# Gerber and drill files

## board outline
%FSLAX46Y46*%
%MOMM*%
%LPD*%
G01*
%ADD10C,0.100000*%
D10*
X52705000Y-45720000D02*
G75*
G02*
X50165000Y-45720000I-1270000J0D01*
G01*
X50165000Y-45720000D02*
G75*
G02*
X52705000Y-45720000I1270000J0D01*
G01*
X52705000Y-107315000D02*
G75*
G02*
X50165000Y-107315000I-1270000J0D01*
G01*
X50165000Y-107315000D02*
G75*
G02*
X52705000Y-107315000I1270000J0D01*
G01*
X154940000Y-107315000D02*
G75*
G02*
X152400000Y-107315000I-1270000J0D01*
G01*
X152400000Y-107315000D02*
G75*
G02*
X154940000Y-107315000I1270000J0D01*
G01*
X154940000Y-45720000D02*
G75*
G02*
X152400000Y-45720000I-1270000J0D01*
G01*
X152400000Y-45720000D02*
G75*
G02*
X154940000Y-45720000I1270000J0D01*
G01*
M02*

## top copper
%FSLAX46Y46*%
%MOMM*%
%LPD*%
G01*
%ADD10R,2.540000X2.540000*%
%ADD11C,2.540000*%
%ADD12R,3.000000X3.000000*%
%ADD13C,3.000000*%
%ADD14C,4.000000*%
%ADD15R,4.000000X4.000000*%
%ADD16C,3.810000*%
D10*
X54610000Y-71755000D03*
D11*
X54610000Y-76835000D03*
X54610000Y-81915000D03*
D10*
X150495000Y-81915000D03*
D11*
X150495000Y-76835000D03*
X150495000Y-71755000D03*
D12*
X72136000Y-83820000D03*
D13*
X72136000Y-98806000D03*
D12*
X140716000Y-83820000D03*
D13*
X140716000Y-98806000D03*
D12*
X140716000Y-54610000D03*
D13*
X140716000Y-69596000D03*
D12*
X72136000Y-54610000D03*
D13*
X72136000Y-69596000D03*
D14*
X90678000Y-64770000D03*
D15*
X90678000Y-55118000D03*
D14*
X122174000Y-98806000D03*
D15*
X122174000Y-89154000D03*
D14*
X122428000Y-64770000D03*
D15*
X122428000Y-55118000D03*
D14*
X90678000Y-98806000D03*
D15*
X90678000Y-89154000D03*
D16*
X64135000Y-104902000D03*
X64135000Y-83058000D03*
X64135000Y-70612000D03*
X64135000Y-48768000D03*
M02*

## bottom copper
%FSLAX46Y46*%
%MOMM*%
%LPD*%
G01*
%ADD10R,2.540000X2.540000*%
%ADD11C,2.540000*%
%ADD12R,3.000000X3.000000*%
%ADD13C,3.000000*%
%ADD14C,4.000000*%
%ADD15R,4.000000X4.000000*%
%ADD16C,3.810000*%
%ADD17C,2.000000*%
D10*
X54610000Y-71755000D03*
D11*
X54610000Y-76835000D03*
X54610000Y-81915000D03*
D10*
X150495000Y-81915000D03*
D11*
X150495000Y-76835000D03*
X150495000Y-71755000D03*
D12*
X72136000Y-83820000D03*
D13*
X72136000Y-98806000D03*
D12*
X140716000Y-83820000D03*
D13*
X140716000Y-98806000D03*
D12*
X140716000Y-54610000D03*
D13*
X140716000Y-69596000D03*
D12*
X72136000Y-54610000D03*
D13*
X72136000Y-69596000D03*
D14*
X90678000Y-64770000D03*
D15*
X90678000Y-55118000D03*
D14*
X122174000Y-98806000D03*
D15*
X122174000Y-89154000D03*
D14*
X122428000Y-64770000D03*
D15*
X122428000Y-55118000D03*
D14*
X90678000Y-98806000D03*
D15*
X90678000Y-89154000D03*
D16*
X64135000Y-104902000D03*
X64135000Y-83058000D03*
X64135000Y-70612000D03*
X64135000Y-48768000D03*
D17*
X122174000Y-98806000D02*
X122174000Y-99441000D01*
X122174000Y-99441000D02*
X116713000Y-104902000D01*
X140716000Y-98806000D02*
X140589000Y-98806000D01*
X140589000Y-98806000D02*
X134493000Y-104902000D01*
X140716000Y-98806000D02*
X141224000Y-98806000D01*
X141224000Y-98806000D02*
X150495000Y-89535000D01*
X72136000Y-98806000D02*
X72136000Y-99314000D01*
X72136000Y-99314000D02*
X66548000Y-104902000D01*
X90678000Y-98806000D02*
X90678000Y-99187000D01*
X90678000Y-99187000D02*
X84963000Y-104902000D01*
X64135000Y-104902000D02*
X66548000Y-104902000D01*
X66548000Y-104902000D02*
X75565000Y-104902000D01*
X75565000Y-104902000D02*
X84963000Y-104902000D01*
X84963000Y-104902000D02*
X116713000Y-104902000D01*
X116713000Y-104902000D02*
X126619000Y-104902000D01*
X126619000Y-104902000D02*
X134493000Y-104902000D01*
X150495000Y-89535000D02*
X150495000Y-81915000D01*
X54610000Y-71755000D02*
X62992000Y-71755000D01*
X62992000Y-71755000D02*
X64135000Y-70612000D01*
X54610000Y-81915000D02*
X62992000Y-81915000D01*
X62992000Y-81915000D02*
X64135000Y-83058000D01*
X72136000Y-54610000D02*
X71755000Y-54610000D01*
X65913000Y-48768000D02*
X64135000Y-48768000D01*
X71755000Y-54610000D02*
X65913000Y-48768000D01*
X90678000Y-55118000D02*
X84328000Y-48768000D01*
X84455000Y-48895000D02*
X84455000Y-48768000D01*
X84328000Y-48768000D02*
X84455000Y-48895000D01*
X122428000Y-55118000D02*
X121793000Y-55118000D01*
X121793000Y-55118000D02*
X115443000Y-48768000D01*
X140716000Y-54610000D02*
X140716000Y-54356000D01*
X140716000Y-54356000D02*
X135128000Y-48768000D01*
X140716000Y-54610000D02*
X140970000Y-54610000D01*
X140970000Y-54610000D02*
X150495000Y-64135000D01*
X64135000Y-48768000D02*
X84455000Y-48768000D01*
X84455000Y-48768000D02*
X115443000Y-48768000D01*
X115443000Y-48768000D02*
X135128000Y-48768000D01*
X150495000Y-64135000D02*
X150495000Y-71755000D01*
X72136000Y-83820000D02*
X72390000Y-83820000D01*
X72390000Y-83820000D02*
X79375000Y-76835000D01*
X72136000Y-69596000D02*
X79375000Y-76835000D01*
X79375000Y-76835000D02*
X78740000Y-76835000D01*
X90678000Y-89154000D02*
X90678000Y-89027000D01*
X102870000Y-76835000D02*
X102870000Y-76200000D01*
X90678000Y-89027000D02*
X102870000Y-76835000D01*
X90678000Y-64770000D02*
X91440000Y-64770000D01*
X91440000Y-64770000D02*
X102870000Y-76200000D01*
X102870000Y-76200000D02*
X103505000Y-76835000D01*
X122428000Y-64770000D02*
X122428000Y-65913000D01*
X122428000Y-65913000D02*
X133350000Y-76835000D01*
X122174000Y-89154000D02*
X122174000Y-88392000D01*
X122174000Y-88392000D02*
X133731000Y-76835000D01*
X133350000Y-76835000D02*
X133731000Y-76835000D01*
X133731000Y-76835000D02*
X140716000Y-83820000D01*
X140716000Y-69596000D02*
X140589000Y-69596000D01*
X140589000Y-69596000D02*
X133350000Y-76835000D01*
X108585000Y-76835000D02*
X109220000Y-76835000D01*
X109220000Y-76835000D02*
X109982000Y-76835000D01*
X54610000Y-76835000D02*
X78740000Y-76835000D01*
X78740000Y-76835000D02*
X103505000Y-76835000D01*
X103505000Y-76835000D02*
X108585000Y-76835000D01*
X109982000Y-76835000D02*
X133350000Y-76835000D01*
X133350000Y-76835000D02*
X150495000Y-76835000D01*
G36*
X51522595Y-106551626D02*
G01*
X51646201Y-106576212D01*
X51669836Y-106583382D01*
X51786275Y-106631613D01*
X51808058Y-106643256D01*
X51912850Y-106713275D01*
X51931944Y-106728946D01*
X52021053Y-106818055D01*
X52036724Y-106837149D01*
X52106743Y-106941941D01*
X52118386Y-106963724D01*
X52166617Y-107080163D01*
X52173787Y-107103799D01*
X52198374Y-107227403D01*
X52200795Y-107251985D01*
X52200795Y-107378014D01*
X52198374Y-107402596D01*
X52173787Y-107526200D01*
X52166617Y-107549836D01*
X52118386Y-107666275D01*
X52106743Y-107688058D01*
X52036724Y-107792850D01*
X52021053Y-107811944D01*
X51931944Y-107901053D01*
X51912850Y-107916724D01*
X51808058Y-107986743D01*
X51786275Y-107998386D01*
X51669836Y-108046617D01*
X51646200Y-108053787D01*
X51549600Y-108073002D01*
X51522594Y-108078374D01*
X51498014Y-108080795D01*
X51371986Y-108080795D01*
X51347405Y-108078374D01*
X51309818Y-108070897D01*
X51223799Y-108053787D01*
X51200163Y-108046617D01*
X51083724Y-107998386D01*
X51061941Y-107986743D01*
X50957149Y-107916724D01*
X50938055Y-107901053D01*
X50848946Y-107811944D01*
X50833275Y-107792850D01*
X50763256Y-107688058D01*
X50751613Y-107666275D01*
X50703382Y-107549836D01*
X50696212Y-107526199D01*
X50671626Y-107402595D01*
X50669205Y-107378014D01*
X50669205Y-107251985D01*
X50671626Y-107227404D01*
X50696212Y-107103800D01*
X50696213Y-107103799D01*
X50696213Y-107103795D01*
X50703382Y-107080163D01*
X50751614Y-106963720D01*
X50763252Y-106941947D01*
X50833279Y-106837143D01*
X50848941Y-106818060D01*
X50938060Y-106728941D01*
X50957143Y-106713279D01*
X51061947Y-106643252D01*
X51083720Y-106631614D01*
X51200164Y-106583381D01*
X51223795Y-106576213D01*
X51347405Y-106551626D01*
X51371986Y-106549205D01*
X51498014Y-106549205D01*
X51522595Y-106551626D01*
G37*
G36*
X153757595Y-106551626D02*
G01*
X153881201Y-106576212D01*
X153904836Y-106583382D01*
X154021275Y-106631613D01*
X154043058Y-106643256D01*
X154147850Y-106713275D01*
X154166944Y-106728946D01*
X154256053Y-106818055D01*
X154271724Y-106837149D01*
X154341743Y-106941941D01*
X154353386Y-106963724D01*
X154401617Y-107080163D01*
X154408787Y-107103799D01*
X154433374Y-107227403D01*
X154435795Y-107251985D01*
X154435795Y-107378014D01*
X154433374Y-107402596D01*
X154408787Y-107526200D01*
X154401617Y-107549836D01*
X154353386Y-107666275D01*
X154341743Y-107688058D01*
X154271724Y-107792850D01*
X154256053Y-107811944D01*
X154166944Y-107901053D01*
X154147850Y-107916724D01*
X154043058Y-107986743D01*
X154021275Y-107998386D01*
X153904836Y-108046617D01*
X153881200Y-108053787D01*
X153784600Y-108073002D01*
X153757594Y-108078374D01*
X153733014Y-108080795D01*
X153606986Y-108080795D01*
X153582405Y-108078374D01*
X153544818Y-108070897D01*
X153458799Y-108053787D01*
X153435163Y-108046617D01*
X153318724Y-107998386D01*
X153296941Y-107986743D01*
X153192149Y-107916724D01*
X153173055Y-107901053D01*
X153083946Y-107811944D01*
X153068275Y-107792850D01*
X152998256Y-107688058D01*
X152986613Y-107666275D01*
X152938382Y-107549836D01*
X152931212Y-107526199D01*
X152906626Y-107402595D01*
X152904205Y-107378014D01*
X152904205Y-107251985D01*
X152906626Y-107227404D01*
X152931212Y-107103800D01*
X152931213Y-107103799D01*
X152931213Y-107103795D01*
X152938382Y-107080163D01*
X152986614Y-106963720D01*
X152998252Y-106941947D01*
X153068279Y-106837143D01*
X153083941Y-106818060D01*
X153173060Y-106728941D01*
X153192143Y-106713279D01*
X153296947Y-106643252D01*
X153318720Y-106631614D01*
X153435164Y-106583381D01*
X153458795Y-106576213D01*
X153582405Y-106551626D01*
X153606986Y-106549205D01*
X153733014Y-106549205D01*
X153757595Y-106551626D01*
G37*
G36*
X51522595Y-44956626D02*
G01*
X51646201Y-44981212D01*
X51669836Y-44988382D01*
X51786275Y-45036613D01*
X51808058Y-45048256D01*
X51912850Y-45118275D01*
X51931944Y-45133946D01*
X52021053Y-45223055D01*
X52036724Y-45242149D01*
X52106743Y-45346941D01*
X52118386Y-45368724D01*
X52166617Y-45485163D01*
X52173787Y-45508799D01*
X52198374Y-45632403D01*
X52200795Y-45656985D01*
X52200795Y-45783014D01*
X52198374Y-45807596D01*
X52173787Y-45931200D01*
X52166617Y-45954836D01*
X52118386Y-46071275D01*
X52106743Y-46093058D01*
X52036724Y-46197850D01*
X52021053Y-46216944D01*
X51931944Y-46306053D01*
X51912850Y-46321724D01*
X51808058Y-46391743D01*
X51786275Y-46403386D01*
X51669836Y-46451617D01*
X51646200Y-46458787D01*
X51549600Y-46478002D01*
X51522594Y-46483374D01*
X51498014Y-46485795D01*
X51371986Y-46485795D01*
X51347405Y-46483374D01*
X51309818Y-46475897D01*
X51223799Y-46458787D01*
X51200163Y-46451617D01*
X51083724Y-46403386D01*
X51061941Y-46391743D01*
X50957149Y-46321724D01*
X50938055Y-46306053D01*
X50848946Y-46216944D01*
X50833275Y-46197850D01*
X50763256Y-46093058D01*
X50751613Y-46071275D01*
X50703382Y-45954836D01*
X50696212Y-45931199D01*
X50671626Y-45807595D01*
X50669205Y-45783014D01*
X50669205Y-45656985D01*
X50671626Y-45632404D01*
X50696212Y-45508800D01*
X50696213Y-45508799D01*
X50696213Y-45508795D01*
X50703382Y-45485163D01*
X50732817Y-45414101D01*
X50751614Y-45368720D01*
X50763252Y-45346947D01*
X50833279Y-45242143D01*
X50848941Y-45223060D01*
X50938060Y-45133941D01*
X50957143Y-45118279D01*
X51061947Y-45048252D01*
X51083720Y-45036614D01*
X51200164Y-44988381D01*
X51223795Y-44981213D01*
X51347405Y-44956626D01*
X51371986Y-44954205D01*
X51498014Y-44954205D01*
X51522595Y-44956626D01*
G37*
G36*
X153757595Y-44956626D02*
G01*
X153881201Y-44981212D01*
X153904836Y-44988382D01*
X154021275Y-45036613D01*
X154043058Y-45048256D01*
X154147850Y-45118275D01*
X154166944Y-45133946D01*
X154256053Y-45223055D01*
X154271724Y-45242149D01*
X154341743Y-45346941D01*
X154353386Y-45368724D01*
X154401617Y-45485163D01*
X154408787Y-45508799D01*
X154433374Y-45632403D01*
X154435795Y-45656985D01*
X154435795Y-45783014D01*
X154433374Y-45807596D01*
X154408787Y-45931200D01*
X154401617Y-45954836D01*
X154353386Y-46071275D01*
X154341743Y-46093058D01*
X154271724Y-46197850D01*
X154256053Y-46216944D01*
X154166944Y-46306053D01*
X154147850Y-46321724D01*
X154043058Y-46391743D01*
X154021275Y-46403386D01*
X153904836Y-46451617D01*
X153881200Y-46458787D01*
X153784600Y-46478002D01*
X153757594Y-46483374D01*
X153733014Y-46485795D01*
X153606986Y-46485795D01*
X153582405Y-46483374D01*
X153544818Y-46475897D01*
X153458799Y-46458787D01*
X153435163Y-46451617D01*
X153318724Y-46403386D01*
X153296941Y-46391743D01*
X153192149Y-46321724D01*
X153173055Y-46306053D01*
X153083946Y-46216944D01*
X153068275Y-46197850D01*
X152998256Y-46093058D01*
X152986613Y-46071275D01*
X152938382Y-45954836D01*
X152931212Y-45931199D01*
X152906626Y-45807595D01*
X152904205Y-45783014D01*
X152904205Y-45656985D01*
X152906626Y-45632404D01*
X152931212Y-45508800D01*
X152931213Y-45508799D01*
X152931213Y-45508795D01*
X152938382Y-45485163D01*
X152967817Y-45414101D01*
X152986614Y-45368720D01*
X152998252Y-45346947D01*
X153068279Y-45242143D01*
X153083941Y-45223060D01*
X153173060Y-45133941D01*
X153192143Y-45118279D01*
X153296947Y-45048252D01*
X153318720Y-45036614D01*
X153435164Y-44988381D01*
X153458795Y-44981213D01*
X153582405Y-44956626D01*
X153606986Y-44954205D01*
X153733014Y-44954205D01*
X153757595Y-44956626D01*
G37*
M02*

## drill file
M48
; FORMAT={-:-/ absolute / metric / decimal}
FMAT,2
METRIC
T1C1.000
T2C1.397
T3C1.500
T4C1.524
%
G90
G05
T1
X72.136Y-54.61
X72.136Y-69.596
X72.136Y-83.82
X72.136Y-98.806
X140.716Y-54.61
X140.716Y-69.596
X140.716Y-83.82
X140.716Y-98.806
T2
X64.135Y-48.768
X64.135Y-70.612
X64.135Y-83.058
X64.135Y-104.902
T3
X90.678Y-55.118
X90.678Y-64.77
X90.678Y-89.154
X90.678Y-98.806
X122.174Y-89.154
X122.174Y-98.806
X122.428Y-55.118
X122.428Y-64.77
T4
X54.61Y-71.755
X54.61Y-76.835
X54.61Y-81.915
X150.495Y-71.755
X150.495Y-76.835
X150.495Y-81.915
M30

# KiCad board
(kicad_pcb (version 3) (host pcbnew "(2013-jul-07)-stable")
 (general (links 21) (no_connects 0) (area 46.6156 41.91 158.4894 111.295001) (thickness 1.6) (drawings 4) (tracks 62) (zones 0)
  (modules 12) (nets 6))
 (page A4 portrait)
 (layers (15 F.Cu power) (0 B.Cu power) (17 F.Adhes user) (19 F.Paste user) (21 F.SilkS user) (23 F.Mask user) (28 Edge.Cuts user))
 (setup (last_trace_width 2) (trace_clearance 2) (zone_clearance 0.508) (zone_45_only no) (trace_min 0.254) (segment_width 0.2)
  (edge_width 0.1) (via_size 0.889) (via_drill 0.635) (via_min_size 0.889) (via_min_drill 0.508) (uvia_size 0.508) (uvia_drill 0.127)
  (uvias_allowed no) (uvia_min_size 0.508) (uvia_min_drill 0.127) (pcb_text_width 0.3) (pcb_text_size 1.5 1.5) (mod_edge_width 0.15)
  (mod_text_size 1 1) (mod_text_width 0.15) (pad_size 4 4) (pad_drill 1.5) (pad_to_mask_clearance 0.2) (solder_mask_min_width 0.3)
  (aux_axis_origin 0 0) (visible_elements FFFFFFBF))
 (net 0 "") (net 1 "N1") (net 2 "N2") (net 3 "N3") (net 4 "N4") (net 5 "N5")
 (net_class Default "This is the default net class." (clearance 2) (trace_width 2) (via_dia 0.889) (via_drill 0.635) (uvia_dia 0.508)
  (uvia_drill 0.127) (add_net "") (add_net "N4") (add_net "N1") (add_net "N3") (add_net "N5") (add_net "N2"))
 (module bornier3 (layer F.Cu) (at 54.61 76.835 270)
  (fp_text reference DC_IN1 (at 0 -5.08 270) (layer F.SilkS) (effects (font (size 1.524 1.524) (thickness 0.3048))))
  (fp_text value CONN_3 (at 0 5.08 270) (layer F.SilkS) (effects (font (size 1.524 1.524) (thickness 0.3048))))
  (pad 1 thru_hole rect (at -5.08 0 270) (size 2.54 2.54) (drill 1.524) (layers *.Cu *.Mask F.SilkS) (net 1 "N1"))
  (pad 2 thru_hole circle (at 0 0 270) (size 2.54 2.54) (drill 1.524) (layers *.Cu *.Mask F.SilkS) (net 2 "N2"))
  (pad 3 thru_hole circle (at 5.08 0 270) (size 2.54 2.54) (drill 1.524) (layers *.Cu *.Mask F.SilkS) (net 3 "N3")))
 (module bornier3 (layer F.Cu) (at 150.495 76.835 90)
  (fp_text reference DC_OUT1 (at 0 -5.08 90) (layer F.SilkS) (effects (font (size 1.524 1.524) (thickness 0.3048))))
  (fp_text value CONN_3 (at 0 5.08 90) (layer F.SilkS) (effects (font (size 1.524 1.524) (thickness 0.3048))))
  (pad 1 thru_hole rect (at -5.08 0 90) (size 2.54 2.54) (drill 1.524) (layers *.Cu *.Mask F.SilkS) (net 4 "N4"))
  (pad 2 thru_hole circle (at 0 0 90) (size 2.54 2.54) (drill 1.524) (layers *.Cu *.Mask F.SilkS) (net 2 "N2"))
  (pad 3 thru_hole circle (at 5.08 0 90) (size 2.54 2.54) (drill 1.524) (layers *.Cu *.Mask F.SilkS) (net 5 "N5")))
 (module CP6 (layer F.Cu) (at 72.136 91.44 270)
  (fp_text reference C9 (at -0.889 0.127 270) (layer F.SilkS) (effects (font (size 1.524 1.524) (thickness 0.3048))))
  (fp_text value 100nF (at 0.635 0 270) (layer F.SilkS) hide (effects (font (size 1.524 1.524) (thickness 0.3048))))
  (pad 1 thru_hole rect (at -7.62 0 270) (size 3 3) (drill 1) (layers *.Cu *.Mask F.SilkS) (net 2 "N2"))
  (pad 2 thru_hole circle (at 7.366 0 270) (size 3 3) (drill 1) (layers *.Cu *.Mask F.SilkS) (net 4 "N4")))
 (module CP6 (layer F.Cu) (at 140.716 91.44 270)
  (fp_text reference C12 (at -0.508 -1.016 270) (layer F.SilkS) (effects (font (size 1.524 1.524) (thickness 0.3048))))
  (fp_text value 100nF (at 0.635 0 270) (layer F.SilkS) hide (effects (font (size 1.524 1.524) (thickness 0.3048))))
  (pad 1 thru_hole rect (at -7.62 0 270) (size 3 3) (drill 1) (layers *.Cu *.Mask F.SilkS) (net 2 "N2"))
  (pad 2 thru_hole circle (at 7.366 0 270) (size 3 3) (drill 1) (layers *.Cu *.Mask F.SilkS) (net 4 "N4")))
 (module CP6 (layer F.Cu) (at 140.716 62.23 270)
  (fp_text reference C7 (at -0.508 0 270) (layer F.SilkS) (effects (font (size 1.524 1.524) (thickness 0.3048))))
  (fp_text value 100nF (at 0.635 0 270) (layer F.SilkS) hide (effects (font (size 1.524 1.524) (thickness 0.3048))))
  (pad 1 thru_hole rect (at -7.62 0 270) (size 3 3) (drill 1) (layers *.Cu *.Mask F.SilkS) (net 5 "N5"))
  (pad 2 thru_hole circle (at 7.366 0 270) (size 3 3) (drill 1) (layers *.Cu *.Mask F.SilkS) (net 2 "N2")))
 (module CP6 (layer F.Cu) (at 72.136 62.23 270)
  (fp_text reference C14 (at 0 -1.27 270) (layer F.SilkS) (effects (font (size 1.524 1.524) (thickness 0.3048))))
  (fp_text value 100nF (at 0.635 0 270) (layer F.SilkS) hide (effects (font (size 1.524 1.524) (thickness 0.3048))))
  (pad 1 thru_hole rect (at -7.62 0 270) (size 3 3) (drill 1) (layers *.Cu *.Mask F.SilkS) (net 5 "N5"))
  (pad 2 thru_hole circle (at 7.366 0 270) (size 3 3) (drill 1) (layers *.Cu *.Mask F.SilkS) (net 2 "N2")))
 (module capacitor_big (layer F.Cu) (at 90.678 59.944 270)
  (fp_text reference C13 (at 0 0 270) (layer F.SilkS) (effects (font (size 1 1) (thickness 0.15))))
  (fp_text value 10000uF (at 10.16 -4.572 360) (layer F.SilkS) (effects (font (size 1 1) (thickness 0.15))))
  (pad 2 thru_hole circle (at 4.826 0 270) (size 4 4) (drill 1.5) (layers *.Cu *.Mask F.SilkS) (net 2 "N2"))
  (pad 1 thru_hole rect (at -4.826 0 270) (size 4 4) (drill 1.5) (layers *.Cu *.Mask F.SilkS) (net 5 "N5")))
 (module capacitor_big (layer F.Cu) (at 122.174 93.98 270)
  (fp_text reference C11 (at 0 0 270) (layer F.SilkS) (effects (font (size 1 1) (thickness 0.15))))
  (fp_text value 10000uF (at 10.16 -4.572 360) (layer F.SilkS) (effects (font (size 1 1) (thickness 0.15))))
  (pad 2 thru_hole circle (at 4.826 0 270) (size 4 4) (drill 1.5) (layers *.Cu *.Mask F.SilkS) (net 4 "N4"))
  (pad 1 thru_hole rect (at -4.826 0 270) (size 4 4) (drill 1.5) (layers *.Cu *.Mask F.SilkS) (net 2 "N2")))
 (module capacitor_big (layer F.Cu) (at 122.428 59.944 270)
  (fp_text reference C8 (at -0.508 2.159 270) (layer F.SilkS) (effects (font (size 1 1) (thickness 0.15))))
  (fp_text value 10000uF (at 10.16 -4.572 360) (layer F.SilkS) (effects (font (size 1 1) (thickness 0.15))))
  (pad 2 thru_hole circle (at 4.826 0 270) (size 4 4) (drill 1.5) (layers *.Cu *.Mask F.SilkS) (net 2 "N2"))
  (pad 1 thru_hole rect (at -4.826 0 270) (size 4 4) (drill 1.5) (layers *.Cu *.Mask F.SilkS) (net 5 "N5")))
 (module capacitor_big (layer F.Cu) (at 90.678 93.98 270)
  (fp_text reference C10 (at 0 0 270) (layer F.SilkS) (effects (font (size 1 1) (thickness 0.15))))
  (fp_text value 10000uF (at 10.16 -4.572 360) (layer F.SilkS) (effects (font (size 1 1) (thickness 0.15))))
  (pad 2 thru_hole circle (at 4.826 0 270) (size 4 4) (drill 1.5) (layers *.Cu *.Mask F.SilkS) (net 4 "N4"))
  (pad 1 thru_hole rect (at -4.826 0 270) (size 4 4) (drill 1.5) (layers *.Cu *.Mask F.SilkS) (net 2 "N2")))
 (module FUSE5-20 (layer F.Cu) (at 64.135 93.98 90)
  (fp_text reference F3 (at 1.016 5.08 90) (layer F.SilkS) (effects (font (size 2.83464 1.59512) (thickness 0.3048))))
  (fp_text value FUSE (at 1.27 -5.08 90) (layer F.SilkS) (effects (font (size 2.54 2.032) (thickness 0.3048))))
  (pad 1 thru_hole circle (at -10.922 0 90) (size 3.81 3.81) (drill 1.397) (layers *.Cu *.Mask F.SilkS) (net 4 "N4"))
  (pad 2 thru_hole circle (at 10.922 0 90) (size 3.81 3.81) (drill 1.397) (layers *.Cu *.Mask F.SilkS) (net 3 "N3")))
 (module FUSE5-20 (layer F.Cu) (at 64.135 59.69 90)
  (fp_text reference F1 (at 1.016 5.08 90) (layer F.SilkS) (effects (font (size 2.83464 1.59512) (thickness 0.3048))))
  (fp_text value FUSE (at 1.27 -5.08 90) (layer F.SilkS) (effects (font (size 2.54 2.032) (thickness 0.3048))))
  (pad 1 thru_hole circle (at -10.922 0 90) (size 3.81 3.81) (drill 1.397) (layers *.Cu *.Mask F.SilkS) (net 1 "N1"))
  (pad 2 thru_hole circle (at 10.922 0 90) (size 3.81 3.81) (drill 1.397) (layers *.Cu *.Mask F.SilkS) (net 5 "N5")))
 (gr_circle (center 51.435 45.72) (end 52.705 45.72) (layer Edge.Cuts) (width 0.1))
 (gr_circle (center 51.435 107.315) (end 52.705 107.315) (layer Edge.Cuts) (width 0.1))
 (gr_circle (center 153.67 107.315) (end 154.94 107.315) (layer Edge.Cuts) (width 0.1))
 (gr_circle (center 153.67 45.72) (end 154.94 45.72) (layer Edge.Cuts) (width 0.1))
 (segment (start 122.174 98.806) (end 122.174 99.441) (width 2) (layer B.Cu) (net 4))
 (segment (start 122.174 99.441) (end 116.713 104.902) (width 2) (layer B.Cu) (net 4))
 (segment (start 140.716 98.806) (end 140.589 98.806) (width 2) (layer B.Cu) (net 4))
 (segment (start 140.589 98.806) (end 134.493 104.902) (width 2) (layer B.Cu) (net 4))
 (segment (start 140.716 98.806) (end 141.224 98.806) (width 2) (layer B.Cu) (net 4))
 (segment (start 141.224 98.806) (end 150.495 89.535) (width 2) (layer B.Cu) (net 4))
 (segment (start 72.136 98.806) (end 72.136 99.314) (width 2) (layer B.Cu) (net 4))
 (segment (start 72.136 99.314) (end 66.548 104.902) (width 2) (layer B.Cu) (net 4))
 (segment (start 90.678 98.806) (end 90.678 99.187) (width 2) (layer B.Cu) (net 4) (status 30))
 (segment (start 90.678 99.187) (end 84.963 104.902) (width 2) (layer B.Cu) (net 4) (status 10))
 (segment (start 64.135 104.902) (end 66.548 104.902) (width 2) (layer B.Cu) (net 4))
 (segment (start 66.548 104.902) (end 75.565 104.902) (width 2) (layer B.Cu) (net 4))
 (segment (start 75.565 104.902) (end 84.963 104.902) (width 2) (layer B.Cu) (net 4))
 (segment (start 84.963 104.902) (end 116.713 104.902) (width 2) (layer B.Cu) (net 4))
 (segment (start 116.713 104.902) (end 126.619 104.902) (width 2) (layer B.Cu) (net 4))
 (segment (start 126.619 104.902) (end 134.493 104.902) (width 2) (layer B.Cu) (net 4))
 (segment (start 150.495 89.535) (end 150.495 81.915) (width 2) (layer B.Cu) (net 4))
 (segment (start 54.61 71.755) (end 62.992 71.755) (width 2) (layer B.Cu) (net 1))
 (segment (start 62.992 71.755) (end 64.135 70.612) (width 2) (layer B.Cu) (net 1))
 (segment (start 54.61 81.915) (end 62.992 81.915) (width 2) (layer B.Cu) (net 3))
 (segment (start 62.992 81.915) (end 64.135 83.058) (width 2) (layer B.Cu) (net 3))
 (segment (start 72.136 54.61) (end 71.755 54.61) (width 2) (layer B.Cu) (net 5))
 (segment (start 65.913 48.768) (end 64.135 48.768) (width 2) (layer B.Cu) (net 5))
 (segment (start 71.755 54.61) (end 65.913 48.768) (width 2) (layer B.Cu) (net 5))
 (segment (start 90.678 55.118) (end 84.328 48.768) (width 2) (layer B.Cu) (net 5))
 (segment (start 84.455 48.895) (end 84.455 48.768) (width 2) (layer B.Cu) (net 5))
 (segment (start 84.328 48.768) (end 84.455 48.895) (width 2) (layer B.Cu) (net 5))
 (segment (start 122.428 55.118) (end 121.793 55.118) (width 2) (layer B.Cu) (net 5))
 (segment (start 121.793 55.118) (end 115.443 48.768) (width 2) (layer B.Cu) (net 5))
 (segment (start 140.716 54.61) (end 140.716 54.356) (width 2) (layer B.Cu) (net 5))
 (segment (start 140.716 54.356) (end 135.128 48.768) (width 2) (layer B.Cu) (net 5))
 (segment (start 140.716 54.61) (end 140.97 54.61) (width 2) (layer B.Cu) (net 5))
 (segment (start 140.97 54.61) (end 150.495 64.135) (width 2) (layer B.Cu) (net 5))
 (segment (start 64.135 48.768) (end 84.455 48.768) (width 2) (layer B.Cu) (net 5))
 (segment (start 84.455 48.768) (end 115.443 48.768) (width 2) (layer B.Cu) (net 5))
 (segment (start 115.443 48.768) (end 135.128 48.768) (width 2) (layer B.Cu) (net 5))
 (segment (start 150.495 64.135) (end 150.495 71.755) (width 2) (layer B.Cu) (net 5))
 (segment (start 72.136 83.82) (end 72.39 83.82) (width 2) (layer B.Cu) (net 2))
 (segment (start 72.39 83.82) (end 79.375 76.835) (width 2) (layer B.Cu) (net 2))
 (segment (start 72.136 69.596) (end 79.375 76.835) (width 2) (layer B.Cu) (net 2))
 (segment (start 79.375 76.835) (end 78.74 76.835) (width 2) (layer B.Cu) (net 2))
 (segment (start 90.678 89.154) (end 90.678 89.027) (width 2) (layer B.Cu) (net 2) (status 30))
 (segment (start 102.87 76.835) (end 102.87 76.2) (width 2) (layer B.Cu) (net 2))
 (segment (start 90.678 89.027) (end 102.87 76.835) (width 2) (layer B.Cu) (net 2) (status 10))
 (segment (start 90.678 64.77) (end 91.44 64.77) (width 2) (layer B.Cu) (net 2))
 (segment (start 91.44 64.77) (end 102.87 76.2) (width 2) (layer B.Cu) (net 2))
 (segment (start 102.87 76.2) (end 103.505 76.835) (width 2) (layer B.Cu) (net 2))
 (segment (start 122.428 64.77) (end 122.428 65.913) (width 2) (layer B.Cu) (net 2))
 (segment (start 122.428 65.913) (end 133.35 76.835) (width 2) (layer B.Cu) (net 2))
 (segment (start 122.174 89.154) (end 122.174 88.392) (width 2) (layer B.Cu) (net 2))
 (segment (start 122.174 88.392) (end 133.731 76.835) (width 2) (layer B.Cu) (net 2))
 (segment (start 133.35 76.835) (end 133.731 76.835) (width 2) (layer B.Cu) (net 2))
 (segment (start 133.731 76.835) (end 140.716 83.82) (width 2) (layer B.Cu) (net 2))
 (segment (start 140.716 69.596) (end 140.589 69.596) (width 2) (layer B.Cu) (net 2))
 (segment (start 140.589 69.596) (end 133.35 76.835) (width 2) (layer B.Cu) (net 2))
 (segment (start 108.585 76.835) (end 109.22 76.835) (width 2) (layer B.Cu) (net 2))
 (segment (start 109.22 76.835) (end 109.982 76.835) (width 2) (layer B.Cu) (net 2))
 (segment (start 54.61 76.835) (end 78.74 76.835) (width 2) (layer B.Cu) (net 2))
 (segment (start 78.74 76.835) (end 103.505 76.835) (width 2) (layer B.Cu) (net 2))
 (segment (start 103.505 76.835) (end 108.585 76.835) (width 2) (layer B.Cu) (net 2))
 (segment (start 109.982 76.835) (end 133.35 76.835) (width 2) (layer B.Cu) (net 2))
 (segment (start 133.35 76.835) (end 150.495 76.835) (width 2) (layer B.Cu) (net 2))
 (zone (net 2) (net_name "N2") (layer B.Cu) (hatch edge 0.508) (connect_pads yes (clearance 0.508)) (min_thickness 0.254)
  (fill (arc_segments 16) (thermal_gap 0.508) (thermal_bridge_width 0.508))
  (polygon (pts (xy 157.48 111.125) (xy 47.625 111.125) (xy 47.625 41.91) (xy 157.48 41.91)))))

